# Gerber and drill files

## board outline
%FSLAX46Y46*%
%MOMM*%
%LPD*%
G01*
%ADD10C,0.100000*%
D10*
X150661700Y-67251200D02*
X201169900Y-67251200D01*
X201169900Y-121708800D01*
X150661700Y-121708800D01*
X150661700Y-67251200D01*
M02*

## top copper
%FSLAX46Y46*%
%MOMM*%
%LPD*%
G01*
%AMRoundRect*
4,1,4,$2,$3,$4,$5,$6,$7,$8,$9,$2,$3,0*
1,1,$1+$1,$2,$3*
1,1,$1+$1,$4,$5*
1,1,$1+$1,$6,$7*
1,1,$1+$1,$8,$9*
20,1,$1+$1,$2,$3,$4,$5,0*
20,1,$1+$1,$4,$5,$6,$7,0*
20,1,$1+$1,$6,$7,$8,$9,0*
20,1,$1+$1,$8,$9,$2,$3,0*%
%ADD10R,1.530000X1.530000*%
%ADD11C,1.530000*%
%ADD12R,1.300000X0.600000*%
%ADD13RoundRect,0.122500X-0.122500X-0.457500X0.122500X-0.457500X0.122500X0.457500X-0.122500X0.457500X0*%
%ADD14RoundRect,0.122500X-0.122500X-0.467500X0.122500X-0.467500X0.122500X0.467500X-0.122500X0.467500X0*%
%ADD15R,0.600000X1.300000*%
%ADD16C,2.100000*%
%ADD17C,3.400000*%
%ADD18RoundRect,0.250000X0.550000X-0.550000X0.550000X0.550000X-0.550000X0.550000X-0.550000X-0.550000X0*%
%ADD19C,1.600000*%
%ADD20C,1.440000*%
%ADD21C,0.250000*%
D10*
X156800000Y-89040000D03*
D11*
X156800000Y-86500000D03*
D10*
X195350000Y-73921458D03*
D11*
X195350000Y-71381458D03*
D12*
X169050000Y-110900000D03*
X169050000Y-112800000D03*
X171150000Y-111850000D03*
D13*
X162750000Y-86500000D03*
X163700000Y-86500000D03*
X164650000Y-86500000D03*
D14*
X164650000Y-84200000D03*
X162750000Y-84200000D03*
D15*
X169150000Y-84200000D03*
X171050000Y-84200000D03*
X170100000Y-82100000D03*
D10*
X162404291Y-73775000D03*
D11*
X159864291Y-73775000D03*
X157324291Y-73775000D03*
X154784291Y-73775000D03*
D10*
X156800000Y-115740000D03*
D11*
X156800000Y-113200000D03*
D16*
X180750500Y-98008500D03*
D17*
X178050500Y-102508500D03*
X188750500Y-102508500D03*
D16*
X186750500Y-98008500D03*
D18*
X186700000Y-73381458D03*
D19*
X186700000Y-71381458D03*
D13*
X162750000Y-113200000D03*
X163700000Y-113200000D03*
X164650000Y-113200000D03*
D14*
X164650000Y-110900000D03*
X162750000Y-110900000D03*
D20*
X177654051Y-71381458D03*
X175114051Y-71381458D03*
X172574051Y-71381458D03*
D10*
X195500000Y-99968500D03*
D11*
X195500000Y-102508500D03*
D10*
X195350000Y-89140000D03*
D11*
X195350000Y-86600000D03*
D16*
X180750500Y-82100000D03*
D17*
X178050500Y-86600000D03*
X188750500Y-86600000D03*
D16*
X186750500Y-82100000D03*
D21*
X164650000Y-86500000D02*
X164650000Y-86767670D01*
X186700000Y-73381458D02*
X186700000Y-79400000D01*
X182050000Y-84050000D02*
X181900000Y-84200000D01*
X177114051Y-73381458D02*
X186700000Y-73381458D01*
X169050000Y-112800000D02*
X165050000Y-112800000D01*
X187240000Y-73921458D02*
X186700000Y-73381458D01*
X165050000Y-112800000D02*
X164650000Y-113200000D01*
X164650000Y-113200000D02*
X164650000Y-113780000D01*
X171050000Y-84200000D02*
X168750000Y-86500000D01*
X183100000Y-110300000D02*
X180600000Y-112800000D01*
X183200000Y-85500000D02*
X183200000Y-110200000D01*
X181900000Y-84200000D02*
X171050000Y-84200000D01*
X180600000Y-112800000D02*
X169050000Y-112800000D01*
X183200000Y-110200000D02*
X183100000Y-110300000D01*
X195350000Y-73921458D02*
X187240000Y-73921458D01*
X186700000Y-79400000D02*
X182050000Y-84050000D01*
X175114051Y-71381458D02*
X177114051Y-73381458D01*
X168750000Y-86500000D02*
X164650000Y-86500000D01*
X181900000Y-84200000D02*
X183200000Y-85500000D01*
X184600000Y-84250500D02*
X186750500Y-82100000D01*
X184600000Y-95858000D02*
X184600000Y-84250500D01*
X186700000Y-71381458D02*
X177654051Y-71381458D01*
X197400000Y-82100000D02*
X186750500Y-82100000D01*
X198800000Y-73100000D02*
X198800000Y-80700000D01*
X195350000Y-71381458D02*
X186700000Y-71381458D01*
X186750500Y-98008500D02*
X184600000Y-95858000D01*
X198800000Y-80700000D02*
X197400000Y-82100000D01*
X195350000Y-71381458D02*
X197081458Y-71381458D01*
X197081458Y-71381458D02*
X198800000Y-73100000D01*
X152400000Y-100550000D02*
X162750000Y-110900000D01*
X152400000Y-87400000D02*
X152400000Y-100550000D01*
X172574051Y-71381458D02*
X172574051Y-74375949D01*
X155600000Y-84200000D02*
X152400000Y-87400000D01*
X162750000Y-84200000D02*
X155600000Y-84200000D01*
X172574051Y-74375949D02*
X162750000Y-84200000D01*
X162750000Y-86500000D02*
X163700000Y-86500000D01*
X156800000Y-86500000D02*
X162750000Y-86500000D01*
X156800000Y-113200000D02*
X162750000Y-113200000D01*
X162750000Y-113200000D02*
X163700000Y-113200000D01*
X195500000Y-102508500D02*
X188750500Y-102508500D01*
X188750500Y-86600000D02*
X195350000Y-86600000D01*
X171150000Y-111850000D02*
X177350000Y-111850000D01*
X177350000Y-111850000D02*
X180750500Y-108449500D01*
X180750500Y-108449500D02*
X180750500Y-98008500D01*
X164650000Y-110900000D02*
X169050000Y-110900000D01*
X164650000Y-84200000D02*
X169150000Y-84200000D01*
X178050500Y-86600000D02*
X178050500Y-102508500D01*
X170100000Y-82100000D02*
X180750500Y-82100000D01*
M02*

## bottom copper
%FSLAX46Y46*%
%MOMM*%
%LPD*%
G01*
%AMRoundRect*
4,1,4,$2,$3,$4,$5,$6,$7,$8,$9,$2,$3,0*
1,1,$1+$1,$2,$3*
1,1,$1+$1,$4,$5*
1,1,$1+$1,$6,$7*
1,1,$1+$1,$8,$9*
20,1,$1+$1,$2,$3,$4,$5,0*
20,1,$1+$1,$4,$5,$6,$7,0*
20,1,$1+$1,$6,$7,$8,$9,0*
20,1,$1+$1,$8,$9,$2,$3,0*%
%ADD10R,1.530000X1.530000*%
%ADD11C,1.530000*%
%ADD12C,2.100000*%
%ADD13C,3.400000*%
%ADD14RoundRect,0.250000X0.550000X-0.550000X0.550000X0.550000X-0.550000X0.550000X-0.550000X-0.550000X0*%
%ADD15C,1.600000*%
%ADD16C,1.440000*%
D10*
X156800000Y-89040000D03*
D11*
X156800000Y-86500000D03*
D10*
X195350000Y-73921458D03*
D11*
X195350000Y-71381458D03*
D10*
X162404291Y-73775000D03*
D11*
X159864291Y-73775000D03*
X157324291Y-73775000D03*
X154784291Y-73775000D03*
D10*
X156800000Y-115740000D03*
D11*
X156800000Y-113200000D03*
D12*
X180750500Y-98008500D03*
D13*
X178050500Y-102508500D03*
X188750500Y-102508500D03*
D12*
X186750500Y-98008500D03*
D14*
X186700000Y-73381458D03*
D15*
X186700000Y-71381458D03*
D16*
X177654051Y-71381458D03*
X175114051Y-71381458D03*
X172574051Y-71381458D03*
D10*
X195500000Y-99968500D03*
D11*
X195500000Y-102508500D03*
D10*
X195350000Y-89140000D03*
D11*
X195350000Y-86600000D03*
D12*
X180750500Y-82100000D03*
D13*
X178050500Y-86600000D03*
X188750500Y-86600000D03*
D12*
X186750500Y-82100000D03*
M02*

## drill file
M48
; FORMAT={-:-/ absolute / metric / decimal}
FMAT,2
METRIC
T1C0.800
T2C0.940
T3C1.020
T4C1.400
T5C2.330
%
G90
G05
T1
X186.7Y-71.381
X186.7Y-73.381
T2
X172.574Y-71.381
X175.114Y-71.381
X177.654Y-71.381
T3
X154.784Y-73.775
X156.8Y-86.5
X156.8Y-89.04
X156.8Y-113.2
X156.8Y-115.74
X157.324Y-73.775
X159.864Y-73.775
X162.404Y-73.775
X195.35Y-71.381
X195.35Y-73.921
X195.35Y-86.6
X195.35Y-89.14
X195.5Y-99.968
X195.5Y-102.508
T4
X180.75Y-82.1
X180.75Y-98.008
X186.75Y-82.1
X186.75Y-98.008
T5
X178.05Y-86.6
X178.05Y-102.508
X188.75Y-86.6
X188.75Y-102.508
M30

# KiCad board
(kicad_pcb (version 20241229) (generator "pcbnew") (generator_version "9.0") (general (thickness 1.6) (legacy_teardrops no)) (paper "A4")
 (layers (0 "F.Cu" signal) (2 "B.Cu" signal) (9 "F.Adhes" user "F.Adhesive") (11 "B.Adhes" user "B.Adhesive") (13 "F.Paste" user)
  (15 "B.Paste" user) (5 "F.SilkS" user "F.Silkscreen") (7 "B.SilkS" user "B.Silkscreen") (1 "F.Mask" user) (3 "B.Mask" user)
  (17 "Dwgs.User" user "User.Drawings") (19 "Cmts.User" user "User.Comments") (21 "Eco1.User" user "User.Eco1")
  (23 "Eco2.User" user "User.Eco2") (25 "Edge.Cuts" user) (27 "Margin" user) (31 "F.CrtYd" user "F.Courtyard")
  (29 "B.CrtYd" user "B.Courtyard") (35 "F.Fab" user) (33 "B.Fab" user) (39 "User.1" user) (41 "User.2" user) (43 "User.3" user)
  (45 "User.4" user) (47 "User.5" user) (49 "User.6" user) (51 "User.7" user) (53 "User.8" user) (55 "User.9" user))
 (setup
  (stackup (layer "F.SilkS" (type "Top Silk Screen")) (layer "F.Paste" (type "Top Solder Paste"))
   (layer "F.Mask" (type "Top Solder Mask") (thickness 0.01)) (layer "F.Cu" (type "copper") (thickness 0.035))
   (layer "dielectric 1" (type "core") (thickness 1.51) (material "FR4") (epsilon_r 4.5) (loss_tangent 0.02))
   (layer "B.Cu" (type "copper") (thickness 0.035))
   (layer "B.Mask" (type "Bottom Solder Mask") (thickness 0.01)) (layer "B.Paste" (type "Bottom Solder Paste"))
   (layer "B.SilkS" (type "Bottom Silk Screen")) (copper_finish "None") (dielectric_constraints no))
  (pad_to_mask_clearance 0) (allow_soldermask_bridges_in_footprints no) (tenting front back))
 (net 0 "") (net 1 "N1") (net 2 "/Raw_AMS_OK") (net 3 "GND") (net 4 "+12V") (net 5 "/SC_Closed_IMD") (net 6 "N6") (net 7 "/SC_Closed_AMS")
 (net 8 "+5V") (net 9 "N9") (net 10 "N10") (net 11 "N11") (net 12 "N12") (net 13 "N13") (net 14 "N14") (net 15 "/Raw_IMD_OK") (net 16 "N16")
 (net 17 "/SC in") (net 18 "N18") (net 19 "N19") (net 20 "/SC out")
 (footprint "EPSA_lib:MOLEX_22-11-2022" (layer "F.Cu") (at 156.8 89.04 90)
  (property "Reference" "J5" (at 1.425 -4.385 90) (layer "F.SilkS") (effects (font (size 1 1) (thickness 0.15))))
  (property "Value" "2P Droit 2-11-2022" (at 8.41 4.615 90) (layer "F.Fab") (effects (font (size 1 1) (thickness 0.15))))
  (pad "1" thru_hole rect (at 0 0 90) (size 1.53 1.53) (drill 1.02) (layers "*.Cu" "*.Mask") (remove_unused_layers no) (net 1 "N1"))
  (pad "2" thru_hole circle (at 2.54 0 90) (size 1.53 1.53) (drill 1.02) (layers "*.Cu" "*.Mask") (remove_unused_layers no)
   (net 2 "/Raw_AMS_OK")))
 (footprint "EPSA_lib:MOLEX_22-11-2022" (layer "F.Cu") (at 195.35 73.921458 90)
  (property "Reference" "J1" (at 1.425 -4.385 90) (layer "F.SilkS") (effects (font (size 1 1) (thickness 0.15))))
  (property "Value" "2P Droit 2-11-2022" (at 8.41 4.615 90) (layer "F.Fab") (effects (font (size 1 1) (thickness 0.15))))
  (pad "1" thru_hole rect (at 0 0 90) (size 1.53 1.53) (drill 1.02) (layers "*.Cu" "*.Mask") (remove_unused_layers no) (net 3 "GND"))
  (pad "2" thru_hole circle (at 2.54 0 90) (size 1.53 1.53) (drill 1.02) (layers "*.Cu" "*.Mask") (remove_unused_layers no) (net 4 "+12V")))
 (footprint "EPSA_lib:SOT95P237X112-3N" (layer "F.Cu") (at 170.1 111.85)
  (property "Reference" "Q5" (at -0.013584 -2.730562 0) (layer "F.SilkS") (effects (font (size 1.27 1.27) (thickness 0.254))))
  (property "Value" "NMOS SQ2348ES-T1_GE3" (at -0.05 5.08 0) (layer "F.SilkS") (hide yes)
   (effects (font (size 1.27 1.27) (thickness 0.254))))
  (pad "1" smd rect (at -1.05 -0.95 90) (size 0.6 1.3) (layers "F.Cu" "F.Mask" "F.Paste") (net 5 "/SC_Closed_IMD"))
  (pad "2" smd rect (at -1.05 0.95 90) (size 0.6 1.3) (layers "F.Cu" "F.Mask" "F.Paste") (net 3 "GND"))
  (pad "3" smd rect (at 1.05 0 90) (size 0.6 1.3) (layers "F.Cu" "F.Mask" "F.Paste") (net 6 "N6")))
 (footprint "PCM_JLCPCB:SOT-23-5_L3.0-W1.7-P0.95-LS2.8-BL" (layer "F.Cu") (at 163.7 85.35)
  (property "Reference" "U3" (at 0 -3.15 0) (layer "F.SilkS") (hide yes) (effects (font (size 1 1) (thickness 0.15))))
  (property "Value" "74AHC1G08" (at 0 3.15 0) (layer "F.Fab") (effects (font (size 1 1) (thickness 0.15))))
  (pad "1" smd roundrect (at -0.95 1.15) (size 0.49 1.16) (layers "F.Cu" "F.Mask" "F.Paste") (roundrect_rratio 0.25) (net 2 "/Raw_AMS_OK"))
  (pad "2" smd roundrect (at 0 1.15) (size 0.49 1.16) (layers "F.Cu" "F.Mask" "F.Paste") (roundrect_rratio 0.25) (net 2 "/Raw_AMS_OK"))
  (pad "3" smd roundrect (at 0.95 1.15) (size 0.49 1.16) (layers "F.Cu" "F.Mask" "F.Paste") (roundrect_rratio 0.25) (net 3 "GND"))
  (pad "4" smd roundrect (at 0.95 -1.15) (size 0.49 1.18) (layers "F.Cu" "F.Mask" "F.Paste") (roundrect_rratio 0.25)
   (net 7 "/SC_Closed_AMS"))
  (pad "5" smd roundrect (at -0.95 -1.15) (size 0.49 1.18) (layers "F.Cu" "F.Mask" "F.Paste") (roundrect_rratio 0.25) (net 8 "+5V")))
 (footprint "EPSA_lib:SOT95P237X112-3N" (layer "F.Cu") (at 170.1 83.15 90)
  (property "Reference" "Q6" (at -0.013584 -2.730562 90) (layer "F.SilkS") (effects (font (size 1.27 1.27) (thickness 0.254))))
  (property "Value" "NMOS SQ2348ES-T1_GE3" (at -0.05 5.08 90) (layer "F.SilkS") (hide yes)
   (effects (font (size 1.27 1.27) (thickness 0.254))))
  (pad "1" smd rect (at -1.05 -0.95 180) (size 0.6 1.3) (layers "F.Cu" "F.Mask" "F.Paste") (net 7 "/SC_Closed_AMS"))
  (pad "2" smd rect (at -1.05 0.95 180) (size 0.6 1.3) (layers "F.Cu" "F.Mask" "F.Paste") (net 3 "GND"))
  (pad "3" smd rect (at 1.05 0 180) (size 0.6 1.3) (layers "F.Cu" "F.Mask" "F.Paste") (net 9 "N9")))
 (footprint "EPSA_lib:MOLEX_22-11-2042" (layer "F.Cu") (at 158.594291 73.775 180)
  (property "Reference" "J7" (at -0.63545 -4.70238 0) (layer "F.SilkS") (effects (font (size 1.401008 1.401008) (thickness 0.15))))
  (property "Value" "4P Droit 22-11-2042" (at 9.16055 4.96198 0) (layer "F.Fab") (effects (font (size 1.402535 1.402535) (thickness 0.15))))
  (pad "1" thru_hole rect (at -3.81 0 180) (size 1.53 1.53) (drill 1.02) (layers "*.Cu" "*.Mask") (remove_unused_layers no) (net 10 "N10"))
  (pad "2" thru_hole circle (at -1.27 0 180) (size 1.53 1.53) (drill 1.02) (layers "*.Cu" "*.Mask") (remove_unused_layers no) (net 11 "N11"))
  (pad "3" thru_hole circle (at 1.27 0 180) (size 1.53 1.53) (drill 1.02) (layers "*.Cu" "*.Mask") (remove_unused_layers no) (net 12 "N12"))
  (pad "4" thru_hole circle (at 3.81 0 180) (size 1.53 1.53) (drill 1.02) (layers "*.Cu" "*.Mask") (remove_unused_layers no) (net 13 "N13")))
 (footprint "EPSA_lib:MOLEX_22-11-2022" (layer "F.Cu") (at 156.8 115.74 90)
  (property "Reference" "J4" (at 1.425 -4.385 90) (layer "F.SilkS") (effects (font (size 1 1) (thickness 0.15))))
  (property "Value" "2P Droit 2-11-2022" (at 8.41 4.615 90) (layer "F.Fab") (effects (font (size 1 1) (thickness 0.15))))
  (pad "1" thru_hole rect (at 0 0 90) (size 1.53 1.53) (drill 1.02) (layers "*.Cu" "*.Mask") (remove_unused_layers no) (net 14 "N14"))
  (pad "2" thru_hole circle (at 2.54 0 90) (size 1.53 1.53) (drill 1.02) (layers "*.Cu" "*.Mask") (remove_unused_layers no)
   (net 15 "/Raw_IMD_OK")))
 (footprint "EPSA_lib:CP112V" (layer "F.Cu") (at 180.7505 98.0085)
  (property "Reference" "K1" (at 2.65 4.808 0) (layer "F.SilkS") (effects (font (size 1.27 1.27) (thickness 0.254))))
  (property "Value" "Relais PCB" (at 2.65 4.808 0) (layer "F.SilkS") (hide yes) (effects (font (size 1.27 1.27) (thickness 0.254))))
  (pad "1" thru_hole circle (at 0 0) (size 2.1 2.1) (drill 1.4) (layers "*.Cu" "*.Mask") (remove_unused_layers no) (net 6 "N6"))
  (pad "2" thru_hole circle (at -2.7 4.5) (size 3.4 3.4) (drill 2.33) (layers "*.Cu" "*.Mask") (remove_unused_layers no) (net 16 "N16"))
  (pad "4" thru_hole circle (at 8 4.5) (size 3.4 3.4) (drill 2.33) (layers "*.Cu" "*.Mask") (remove_unused_layers no) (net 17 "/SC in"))
  (pad "5" thru_hole circle (at 6 0) (size 2.1 2.1) (drill 1.4) (layers "*.Cu" "*.Mask") (remove_unused_layers no) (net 4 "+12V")))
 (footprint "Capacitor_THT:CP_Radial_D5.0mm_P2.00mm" (layer "F.Cu") (at 186.7 73.381458 90)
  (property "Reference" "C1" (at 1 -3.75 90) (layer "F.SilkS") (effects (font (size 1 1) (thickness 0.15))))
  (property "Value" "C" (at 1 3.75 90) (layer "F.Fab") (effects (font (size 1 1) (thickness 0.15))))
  (pad "1" thru_hole roundrect (at 0 0 90) (size 1.6 1.6) (drill 0.8) (layers "*.Cu" "*.Mask") (remove_unused_layers no)
   (roundrect_rratio 0.15625) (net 3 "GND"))
  (pad "2" thru_hole circle (at 2 0 90) (size 1.6 1.6) (drill 0.8) (layers "*.Cu" "*.Mask") (remove_unused_layers no) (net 4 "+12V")))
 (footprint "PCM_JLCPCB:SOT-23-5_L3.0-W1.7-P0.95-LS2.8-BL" (layer "F.Cu") (at 163.7 112.05)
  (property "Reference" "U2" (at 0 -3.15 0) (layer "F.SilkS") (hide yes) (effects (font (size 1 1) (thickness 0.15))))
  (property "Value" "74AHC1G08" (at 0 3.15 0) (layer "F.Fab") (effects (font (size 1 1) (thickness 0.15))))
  (pad "1" smd roundrect (at -0.95 1.15) (size 0.49 1.16) (layers "F.Cu" "F.Mask" "F.Paste") (roundrect_rratio 0.25) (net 15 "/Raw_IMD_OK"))
  (pad "2" smd roundrect (at 0 1.15) (size 0.49 1.16) (layers "F.Cu" "F.Mask" "F.Paste") (roundrect_rratio 0.25) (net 15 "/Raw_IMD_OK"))
  (pad "3" smd roundrect (at 0.95 1.15) (size 0.49 1.16) (layers "F.Cu" "F.Mask" "F.Paste") (roundrect_rratio 0.25) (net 3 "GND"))
  (pad "4" smd roundrect (at 0.95 -1.15) (size 0.49 1.18) (layers "F.Cu" "F.Mask" "F.Paste") (roundrect_rratio 0.25)
   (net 5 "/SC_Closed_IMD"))
  (pad "5" smd roundrect (at -0.95 -1.15) (size 0.49 1.18) (layers "F.Cu" "F.Mask" "F.Paste") (roundrect_rratio 0.25) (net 8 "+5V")))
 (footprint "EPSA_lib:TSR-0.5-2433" (layer "F.Cu") (at 180.864051 69.381458 180)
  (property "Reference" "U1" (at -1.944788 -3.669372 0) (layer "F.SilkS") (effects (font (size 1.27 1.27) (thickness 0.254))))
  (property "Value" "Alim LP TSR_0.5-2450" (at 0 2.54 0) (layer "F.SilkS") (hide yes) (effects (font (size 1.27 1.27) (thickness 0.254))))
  (pad "1" thru_hole circle (at 3.21 -2 180) (size 1.44 1.44) (drill 0.94) (layers "*.Cu" "*.Mask") (remove_unused_layers no) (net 4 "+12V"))
  (pad "2" thru_hole circle (at 5.75 -2 180) (size 1.44 1.44) (drill 0.94) (layers "*.Cu" "*.Mask") (remove_unused_layers no) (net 3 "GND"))
  (pad "3" thru_hole circle (at 8.29 -2 180) (size 1.44 1.44) (drill 0.94) (layers "*.Cu" "*.Mask") (remove_unused_layers no) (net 8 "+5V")))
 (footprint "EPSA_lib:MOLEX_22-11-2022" (layer "F.Cu") (at 195.5 99.9685 -90)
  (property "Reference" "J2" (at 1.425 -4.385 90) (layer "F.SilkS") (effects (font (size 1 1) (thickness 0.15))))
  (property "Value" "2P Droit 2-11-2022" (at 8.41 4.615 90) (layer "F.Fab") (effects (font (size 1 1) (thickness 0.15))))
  (pad "1" thru_hole rect (at 0 0 270) (size 1.53 1.53) (drill 1.02) (layers "*.Cu" "*.Mask") (remove_unused_layers no) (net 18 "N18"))
  (pad "2" thru_hole circle (at 2.54 0 270) (size 1.53 1.53) (drill 1.02) (layers "*.Cu" "*.Mask") (remove_unused_layers no)
   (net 17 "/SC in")))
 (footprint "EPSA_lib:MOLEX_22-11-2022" (layer "F.Cu") (at 195.35 89.14 90)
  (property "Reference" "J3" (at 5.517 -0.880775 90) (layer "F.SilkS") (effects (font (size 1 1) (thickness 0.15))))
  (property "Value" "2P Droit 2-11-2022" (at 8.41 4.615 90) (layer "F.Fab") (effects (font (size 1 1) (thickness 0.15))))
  (pad "1" thru_hole rect (at 0 0 90) (size 1.53 1.53) (drill 1.02) (layers "*.Cu" "*.Mask") (remove_unused_layers no) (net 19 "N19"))
  (pad "2" thru_hole circle (at 2.54 0 90) (size 1.53 1.53) (drill 1.02) (layers "*.Cu" "*.Mask") (remove_unused_layers no)
   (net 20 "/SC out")))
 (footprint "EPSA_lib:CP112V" (layer "F.Cu") (at 180.7505 82.1)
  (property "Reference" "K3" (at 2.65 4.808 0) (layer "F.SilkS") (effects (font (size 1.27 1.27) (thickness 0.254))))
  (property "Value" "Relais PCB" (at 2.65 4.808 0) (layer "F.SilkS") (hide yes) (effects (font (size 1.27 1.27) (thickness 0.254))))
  (pad "1" thru_hole circle (at 0 0) (size 2.1 2.1) (drill 1.4) (layers "*.Cu" "*.Mask") (remove_unused_layers no) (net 9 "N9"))
  (pad "2" thru_hole circle (at -2.7 4.5) (size 3.4 3.4) (drill 2.33) (layers "*.Cu" "*.Mask") (remove_unused_layers no) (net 16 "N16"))
  (pad "4" thru_hole circle (at 8 4.5) (size 3.4 3.4) (drill 2.33) (layers "*.Cu" "*.Mask") (remove_unused_layers no) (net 20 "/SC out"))
  (pad "5" thru_hole circle (at 6 0) (size 2.1 2.1) (drill 1.4) (layers "*.Cu" "*.Mask") (remove_unused_layers no) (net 4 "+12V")))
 (gr_rect (start 150.6617 67.2512) (end 201.1699 121.7088) (stroke (width 0.1) (type default)) (fill no) (layer "Edge.Cuts"))
 (segment (start 164.65 86.5) (end 164.65 86.76767) (width 0.25) (layer "F.Cu") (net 3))
 (segment (start 186.7 73.381458) (end 186.7 79.4) (width 0.25) (layer "F.Cu") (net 3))
 (segment (start 182.05 84.05) (end 181.9 84.2) (width 0.25) (layer "F.Cu") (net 3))
 (segment (start 177.114051 73.381458) (end 186.7 73.381458) (width 0.25) (layer "F.Cu") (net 3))
 (segment (start 169.05 112.8) (end 165.05 112.8) (width 0.25) (layer "F.Cu") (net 3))
 (segment (start 187.24 73.921458) (end 186.7 73.381458) (width 0.25) (layer "F.Cu") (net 3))
 (segment (start 165.05 112.8) (end 164.65 113.2) (width 0.25) (layer "F.Cu") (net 3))
 (segment (start 164.65 113.2) (end 164.65 113.78) (width 0.25) (layer "F.Cu") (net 3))
 (segment (start 171.05 84.2) (end 168.75 86.5) (width 0.25) (layer "F.Cu") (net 3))
 (segment (start 183.1 110.3) (end 180.6 112.8) (width 0.25) (layer "F.Cu") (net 3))
 (segment (start 183.2 85.5) (end 183.2 110.2) (width 0.25) (layer "F.Cu") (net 3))
 (segment (start 181.9 84.2) (end 171.05 84.2) (width 0.25) (layer "F.Cu") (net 3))
 (segment (start 180.6 112.8) (end 169.05 112.8) (width 0.25) (layer "F.Cu") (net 3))
 (segment (start 183.2 110.2) (end 183.1 110.3) (width 0.25) (layer "F.Cu") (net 3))
 (segment (start 195.35 73.921458) (end 187.24 73.921458) (width 0.25) (layer "F.Cu") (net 3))
 (segment (start 186.7 79.4) (end 182.05 84.05) (width 0.25) (layer "F.Cu") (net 3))
 (segment (start 175.114051 71.381458) (end 177.114051 73.381458) (width 0.25) (layer "F.Cu") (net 3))
 (segment (start 168.75 86.5) (end 164.65 86.5) (width 0.25) (layer "F.Cu") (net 3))
 (segment (start 181.9 84.2) (end 183.2 85.5) (width 0.25) (layer "F.Cu") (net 3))
 (segment (start 184.6 84.2505) (end 186.7505 82.1) (width 0.25) (layer "F.Cu") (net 4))
 (segment (start 184.6 95.858) (end 184.6 84.2505) (width 0.25) (layer "F.Cu") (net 4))
 (segment (start 186.7 71.381458) (end 177.654051 71.381458) (width 0.25) (layer "F.Cu") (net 4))
 (segment (start 197.4 82.1) (end 186.7505 82.1) (width 0.25) (layer "F.Cu") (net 4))
 (segment (start 198.8 73.1) (end 198.8 80.7) (width 0.25) (layer "F.Cu") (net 4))
 (segment (start 195.35 71.381458) (end 186.7 71.381458) (width 0.25) (layer "F.Cu") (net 4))
 (segment (start 186.7505 98.0085) (end 184.6 95.858) (width 0.25) (layer "F.Cu") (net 4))
 (segment (start 198.8 80.7) (end 197.4 82.1) (width 0.25) (layer "F.Cu") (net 4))
 (segment (start 195.35 71.381458) (end 197.081458 71.381458) (width 0.25) (layer "F.Cu") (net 4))
 (segment (start 197.081458 71.381458) (end 198.8 73.1) (width 0.25) (layer "F.Cu") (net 4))
 (segment (start 152.4 100.55) (end 162.75 110.9) (width 0.25) (layer "F.Cu") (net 8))
 (segment (start 152.4 87.4) (end 152.4 100.55) (width 0.25) (layer "F.Cu") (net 8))
 (segment (start 172.574051 71.381458) (end 172.574051 74.375949) (width 0.25) (layer "F.Cu") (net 8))
 (segment (start 155.6 84.2) (end 152.4 87.4) (width 0.25) (layer "F.Cu") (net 8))
 (segment (start 162.75 84.2) (end 155.6 84.2) (width 0.25) (layer "F.Cu") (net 8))
 (segment (start 172.574051 74.375949) (end 162.75 84.2) (width 0.25) (layer "F.Cu") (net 8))
 (segment (start 162.75 86.5) (end 163.7 86.5) (width 0.25) (layer "F.Cu") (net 2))
 (segment (start 156.8 86.5) (end 162.75 86.5) (width 0.25) (layer "F.Cu") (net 2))
 (segment (start 156.8 113.2) (end 162.75 113.2) (width 0.25) (layer "F.Cu") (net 15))
 (segment (start 162.75 113.2) (end 163.7 113.2) (width 0.25) (layer "F.Cu") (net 15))
 (segment (start 195.5 102.5085) (end 188.7505 102.5085) (width 0.25) (layer "F.Cu") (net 17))
 (segment (start 188.7505 86.6) (end 195.35 86.6) (width 0.25) (layer "F.Cu") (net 20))
 (segment (start 171.15 111.85) (end 177.35 111.85) (width 0.25) (layer "F.Cu") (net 6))
 (segment (start 177.35 111.85) (end 180.7505 108.4495) (width 0.25) (layer "F.Cu") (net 6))
 (segment (start 180.7505 108.4495) (end 180.7505 98.0085) (width 0.25) (layer "F.Cu") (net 6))
 (segment (start 164.65 110.9) (end 169.05 110.9) (width 0.25) (layer "F.Cu") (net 5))
 (segment (start 164.65 84.2) (end 169.15 84.2) (width 0.25) (layer "F.Cu") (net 7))
 (segment (start 178.0505 86.6) (end 178.0505 102.5085) (width 0.25) (layer "F.Cu") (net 16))
 (segment (start 170.1 82.1) (end 180.7505 82.1) (width 0.25) (layer "F.Cu") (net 9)))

